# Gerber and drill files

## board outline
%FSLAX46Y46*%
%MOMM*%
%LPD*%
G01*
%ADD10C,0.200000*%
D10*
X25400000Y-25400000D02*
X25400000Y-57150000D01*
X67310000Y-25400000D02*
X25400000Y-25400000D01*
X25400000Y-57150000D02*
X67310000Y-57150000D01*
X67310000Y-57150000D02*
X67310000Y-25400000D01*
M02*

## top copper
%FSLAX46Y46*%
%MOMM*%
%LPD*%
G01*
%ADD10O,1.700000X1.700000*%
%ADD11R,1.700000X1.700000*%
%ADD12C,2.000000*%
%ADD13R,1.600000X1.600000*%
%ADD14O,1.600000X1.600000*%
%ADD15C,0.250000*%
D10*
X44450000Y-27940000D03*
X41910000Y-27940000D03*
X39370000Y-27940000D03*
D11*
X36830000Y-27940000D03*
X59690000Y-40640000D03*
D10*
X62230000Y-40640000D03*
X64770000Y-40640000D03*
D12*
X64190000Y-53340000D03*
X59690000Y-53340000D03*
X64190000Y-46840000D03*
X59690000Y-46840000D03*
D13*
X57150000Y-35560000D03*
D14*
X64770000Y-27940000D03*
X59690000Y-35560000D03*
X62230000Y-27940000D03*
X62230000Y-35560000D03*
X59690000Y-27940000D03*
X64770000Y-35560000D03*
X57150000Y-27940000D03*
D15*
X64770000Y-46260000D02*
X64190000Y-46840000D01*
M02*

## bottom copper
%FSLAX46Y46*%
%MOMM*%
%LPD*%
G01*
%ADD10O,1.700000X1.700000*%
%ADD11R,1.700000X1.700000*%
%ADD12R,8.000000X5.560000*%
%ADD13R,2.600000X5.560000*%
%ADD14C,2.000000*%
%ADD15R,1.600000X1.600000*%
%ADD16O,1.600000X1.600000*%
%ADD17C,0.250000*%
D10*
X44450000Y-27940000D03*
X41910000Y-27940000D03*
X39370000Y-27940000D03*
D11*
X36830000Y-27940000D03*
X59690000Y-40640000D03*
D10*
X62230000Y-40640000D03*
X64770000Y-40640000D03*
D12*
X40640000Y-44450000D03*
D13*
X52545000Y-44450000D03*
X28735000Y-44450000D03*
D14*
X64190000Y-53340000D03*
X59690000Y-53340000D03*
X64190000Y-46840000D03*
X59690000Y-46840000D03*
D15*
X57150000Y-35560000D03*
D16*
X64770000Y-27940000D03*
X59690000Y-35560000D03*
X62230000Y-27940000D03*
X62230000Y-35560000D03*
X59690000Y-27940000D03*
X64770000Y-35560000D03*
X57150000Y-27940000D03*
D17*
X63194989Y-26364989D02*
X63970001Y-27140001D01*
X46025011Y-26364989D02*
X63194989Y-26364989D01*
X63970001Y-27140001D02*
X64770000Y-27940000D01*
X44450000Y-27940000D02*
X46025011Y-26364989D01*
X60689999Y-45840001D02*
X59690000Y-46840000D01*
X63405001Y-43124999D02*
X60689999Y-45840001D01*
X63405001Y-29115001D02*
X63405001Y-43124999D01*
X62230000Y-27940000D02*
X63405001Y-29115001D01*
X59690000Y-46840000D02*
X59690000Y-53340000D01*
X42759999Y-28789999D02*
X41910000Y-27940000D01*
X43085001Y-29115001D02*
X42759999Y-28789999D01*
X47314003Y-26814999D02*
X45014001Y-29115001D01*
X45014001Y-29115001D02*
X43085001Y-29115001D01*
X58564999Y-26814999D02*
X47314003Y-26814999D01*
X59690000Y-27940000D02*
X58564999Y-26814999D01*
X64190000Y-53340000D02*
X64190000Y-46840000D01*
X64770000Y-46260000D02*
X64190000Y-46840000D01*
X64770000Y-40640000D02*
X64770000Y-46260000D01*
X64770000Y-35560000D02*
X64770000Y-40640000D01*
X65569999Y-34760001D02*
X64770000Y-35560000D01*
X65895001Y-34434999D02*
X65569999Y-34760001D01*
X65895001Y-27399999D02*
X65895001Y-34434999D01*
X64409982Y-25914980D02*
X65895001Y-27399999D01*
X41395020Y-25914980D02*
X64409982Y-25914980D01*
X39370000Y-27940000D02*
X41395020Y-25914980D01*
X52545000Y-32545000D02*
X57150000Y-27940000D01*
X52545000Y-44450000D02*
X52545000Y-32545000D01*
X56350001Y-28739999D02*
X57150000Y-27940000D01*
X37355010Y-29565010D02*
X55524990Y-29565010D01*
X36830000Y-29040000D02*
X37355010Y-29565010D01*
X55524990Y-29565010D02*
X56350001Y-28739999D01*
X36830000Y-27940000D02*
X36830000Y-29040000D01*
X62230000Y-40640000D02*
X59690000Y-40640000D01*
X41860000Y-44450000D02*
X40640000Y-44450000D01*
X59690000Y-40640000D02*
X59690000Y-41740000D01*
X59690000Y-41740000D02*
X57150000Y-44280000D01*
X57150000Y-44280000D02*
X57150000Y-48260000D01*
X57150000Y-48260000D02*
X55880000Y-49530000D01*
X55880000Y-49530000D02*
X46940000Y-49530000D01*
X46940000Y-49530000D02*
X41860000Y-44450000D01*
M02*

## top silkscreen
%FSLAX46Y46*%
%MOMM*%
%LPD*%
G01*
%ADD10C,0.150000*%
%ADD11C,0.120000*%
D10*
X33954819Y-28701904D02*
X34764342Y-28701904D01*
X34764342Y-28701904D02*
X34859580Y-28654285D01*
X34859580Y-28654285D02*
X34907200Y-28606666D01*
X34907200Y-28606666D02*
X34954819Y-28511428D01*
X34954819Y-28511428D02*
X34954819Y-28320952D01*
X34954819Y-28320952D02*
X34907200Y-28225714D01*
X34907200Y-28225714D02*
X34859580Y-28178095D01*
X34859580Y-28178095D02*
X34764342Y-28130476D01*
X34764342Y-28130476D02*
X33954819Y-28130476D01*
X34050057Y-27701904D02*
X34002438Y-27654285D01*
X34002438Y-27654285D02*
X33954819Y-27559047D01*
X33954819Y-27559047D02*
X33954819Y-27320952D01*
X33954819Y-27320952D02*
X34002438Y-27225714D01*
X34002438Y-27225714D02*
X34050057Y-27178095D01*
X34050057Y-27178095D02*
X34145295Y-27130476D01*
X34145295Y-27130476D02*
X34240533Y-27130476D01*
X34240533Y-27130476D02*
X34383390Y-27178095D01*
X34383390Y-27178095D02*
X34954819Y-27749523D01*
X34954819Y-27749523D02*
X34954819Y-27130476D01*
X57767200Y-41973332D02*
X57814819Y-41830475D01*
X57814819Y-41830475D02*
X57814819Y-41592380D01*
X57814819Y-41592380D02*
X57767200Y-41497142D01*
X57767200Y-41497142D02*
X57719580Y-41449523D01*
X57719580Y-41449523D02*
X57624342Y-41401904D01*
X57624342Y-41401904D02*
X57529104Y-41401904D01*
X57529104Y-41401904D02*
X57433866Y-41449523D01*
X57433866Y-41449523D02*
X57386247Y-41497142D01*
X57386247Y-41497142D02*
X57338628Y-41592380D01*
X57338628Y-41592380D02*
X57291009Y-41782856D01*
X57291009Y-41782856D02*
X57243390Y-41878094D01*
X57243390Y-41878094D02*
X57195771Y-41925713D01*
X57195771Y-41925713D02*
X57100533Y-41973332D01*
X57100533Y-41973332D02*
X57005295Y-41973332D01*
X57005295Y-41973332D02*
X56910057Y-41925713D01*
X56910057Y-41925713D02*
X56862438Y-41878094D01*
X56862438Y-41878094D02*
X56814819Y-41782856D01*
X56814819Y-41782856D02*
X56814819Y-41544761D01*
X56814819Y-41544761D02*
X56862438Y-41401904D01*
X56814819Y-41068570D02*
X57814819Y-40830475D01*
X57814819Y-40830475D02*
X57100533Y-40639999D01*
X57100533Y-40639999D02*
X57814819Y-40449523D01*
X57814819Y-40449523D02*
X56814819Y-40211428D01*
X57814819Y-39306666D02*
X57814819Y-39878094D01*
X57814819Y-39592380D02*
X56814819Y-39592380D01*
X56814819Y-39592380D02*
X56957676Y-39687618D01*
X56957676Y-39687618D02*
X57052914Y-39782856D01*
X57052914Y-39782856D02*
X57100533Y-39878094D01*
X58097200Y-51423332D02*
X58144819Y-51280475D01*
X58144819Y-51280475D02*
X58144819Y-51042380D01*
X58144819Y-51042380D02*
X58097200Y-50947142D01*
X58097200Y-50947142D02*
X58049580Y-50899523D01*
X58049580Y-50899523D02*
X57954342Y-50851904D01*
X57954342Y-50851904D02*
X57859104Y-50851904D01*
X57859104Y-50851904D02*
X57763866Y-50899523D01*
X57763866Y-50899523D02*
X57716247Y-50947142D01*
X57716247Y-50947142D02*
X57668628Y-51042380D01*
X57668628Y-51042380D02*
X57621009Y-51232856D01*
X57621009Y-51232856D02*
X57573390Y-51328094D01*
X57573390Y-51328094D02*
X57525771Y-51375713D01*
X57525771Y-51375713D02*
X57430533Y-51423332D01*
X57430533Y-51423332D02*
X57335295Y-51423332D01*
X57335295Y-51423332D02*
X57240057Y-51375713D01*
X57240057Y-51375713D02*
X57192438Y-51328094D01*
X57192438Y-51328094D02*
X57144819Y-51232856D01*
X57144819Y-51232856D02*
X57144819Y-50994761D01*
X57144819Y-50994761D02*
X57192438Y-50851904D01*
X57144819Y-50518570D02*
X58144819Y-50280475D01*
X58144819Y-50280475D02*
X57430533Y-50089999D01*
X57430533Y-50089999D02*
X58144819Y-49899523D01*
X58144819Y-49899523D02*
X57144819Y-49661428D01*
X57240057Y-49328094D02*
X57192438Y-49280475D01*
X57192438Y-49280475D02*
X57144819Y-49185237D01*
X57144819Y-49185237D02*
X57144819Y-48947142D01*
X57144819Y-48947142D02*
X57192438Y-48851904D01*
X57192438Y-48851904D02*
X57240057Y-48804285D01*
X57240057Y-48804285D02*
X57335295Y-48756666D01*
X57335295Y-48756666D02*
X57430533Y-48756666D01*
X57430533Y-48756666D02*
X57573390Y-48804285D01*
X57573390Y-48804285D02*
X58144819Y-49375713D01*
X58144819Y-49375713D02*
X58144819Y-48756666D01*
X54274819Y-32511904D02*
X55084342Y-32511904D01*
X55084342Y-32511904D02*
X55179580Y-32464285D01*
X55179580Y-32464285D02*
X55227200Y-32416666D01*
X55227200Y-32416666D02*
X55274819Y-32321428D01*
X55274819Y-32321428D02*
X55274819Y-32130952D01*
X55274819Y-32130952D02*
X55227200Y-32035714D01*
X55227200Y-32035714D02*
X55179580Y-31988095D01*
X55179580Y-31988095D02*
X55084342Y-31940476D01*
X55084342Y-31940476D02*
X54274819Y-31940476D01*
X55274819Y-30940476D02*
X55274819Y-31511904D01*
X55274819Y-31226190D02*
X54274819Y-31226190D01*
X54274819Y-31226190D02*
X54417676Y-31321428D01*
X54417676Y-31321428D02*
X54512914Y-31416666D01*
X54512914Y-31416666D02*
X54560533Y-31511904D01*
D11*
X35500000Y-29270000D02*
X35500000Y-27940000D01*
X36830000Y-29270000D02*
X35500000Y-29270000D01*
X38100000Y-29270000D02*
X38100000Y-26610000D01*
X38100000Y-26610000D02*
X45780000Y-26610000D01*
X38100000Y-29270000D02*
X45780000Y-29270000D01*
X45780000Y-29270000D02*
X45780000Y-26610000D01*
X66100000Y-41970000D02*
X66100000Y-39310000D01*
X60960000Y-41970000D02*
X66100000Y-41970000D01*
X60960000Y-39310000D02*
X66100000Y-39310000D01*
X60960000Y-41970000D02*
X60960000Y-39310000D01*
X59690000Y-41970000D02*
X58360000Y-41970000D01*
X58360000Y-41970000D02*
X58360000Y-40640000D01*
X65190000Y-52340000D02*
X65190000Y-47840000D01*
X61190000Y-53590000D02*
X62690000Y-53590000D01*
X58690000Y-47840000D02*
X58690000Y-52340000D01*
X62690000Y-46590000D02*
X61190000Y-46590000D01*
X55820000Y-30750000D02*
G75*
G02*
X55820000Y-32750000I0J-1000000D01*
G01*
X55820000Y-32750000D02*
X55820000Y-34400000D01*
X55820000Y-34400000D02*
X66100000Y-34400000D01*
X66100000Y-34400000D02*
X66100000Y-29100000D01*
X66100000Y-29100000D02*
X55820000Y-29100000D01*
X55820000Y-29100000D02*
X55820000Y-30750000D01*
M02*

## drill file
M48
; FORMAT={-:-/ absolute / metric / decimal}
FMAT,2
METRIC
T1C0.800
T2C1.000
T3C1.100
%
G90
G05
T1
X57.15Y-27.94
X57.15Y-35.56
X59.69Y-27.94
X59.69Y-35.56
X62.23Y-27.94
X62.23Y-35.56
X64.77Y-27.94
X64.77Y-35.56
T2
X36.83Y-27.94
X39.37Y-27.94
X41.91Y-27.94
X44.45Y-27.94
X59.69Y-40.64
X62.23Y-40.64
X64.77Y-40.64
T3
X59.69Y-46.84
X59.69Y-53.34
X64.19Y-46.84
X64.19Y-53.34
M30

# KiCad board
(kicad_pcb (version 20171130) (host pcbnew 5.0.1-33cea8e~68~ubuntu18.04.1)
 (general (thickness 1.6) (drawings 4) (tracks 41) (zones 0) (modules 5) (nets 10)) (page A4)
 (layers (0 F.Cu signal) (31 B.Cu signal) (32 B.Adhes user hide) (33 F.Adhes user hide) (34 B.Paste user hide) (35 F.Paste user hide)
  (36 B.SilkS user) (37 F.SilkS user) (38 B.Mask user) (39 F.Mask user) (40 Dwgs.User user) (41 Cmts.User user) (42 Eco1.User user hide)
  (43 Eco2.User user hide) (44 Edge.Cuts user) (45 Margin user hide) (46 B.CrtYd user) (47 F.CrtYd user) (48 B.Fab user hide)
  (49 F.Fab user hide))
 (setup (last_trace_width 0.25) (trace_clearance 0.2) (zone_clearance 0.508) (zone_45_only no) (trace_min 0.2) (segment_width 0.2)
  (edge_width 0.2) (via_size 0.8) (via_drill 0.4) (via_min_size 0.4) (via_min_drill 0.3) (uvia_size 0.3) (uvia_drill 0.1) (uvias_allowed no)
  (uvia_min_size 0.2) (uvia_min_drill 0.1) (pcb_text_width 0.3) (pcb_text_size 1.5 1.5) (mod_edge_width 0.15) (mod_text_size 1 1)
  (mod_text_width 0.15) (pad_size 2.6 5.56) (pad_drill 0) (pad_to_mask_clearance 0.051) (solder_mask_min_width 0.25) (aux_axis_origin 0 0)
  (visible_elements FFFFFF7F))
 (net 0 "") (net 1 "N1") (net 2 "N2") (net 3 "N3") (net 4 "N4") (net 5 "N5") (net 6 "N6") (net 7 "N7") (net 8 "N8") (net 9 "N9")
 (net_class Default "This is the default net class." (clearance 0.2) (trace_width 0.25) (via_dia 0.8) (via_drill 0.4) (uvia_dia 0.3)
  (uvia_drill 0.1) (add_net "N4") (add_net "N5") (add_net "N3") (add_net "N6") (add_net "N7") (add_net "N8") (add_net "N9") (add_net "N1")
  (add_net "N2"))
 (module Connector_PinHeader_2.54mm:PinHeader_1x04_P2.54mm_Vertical (layer F.Cu) (at 36.83 27.94 90)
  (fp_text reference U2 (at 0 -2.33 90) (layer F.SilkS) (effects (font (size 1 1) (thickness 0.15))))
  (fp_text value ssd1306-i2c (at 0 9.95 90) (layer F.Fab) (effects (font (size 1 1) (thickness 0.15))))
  (fp_line (start -1.33 -1.33) (end 0 -1.33) (layer F.SilkS) (width 0.12))
  (fp_line (start -1.33 0) (end -1.33 -1.33) (layer F.SilkS) (width 0.12))
  (fp_line (start -1.33 1.27) (end 1.33 1.27) (layer F.SilkS) (width 0.12))
  (fp_line (start 1.33 1.27) (end 1.33 8.95) (layer F.SilkS) (width 0.12))
  (fp_line (start -1.33 1.27) (end -1.33 8.95) (layer F.SilkS) (width 0.12))
  (fp_line (start -1.33 8.95) (end 1.33 8.95) (layer F.SilkS) (width 0.12))
  (pad 4 thru_hole oval (at 0 7.62 90) (size 1.7 1.7) (drill 1) (layers *.Cu *.Mask) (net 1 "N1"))
  (pad 3 thru_hole oval (at 0 5.08 90) (size 1.7 1.7) (drill 1) (layers *.Cu *.Mask) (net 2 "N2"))
  (pad 2 thru_hole oval (at 0 2.54 90) (size 1.7 1.7) (drill 1) (layers *.Cu *.Mask) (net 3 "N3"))
  (pad 1 thru_hole rect (at 0 0 90) (size 1.7 1.7) (drill 1) (layers *.Cu *.Mask) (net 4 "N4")))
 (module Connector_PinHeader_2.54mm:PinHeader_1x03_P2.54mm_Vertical (layer F.Cu) (at 59.69 40.64 90)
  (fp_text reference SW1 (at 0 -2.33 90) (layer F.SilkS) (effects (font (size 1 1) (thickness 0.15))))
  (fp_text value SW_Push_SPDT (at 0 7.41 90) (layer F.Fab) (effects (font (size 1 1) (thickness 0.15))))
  (fp_line (start -1.33 6.41) (end 1.33 6.41) (layer F.SilkS) (width 0.12))
  (fp_line (start -1.33 1.27) (end -1.33 6.41) (layer F.SilkS) (width 0.12))
  (fp_line (start 1.33 1.27) (end 1.33 6.41) (layer F.SilkS) (width 0.12))
  (fp_line (start -1.33 1.27) (end 1.33 1.27) (layer F.SilkS) (width 0.12))
  (fp_line (start -1.33 0) (end -1.33 -1.33) (layer F.SilkS) (width 0.12))
  (fp_line (start -1.33 -1.33) (end 0 -1.33) (layer F.SilkS) (width 0.12))
  (pad 1 thru_hole rect (at 0 0 90) (size 1.7 1.7) (drill 1) (layers *.Cu *.Mask) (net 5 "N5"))
  (pad 2 thru_hole oval (at 0 2.54 90) (size 1.7 1.7) (drill 1) (layers *.Cu *.Mask) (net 5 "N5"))
  (pad 3 thru_hole oval (at 0 5.08 90) (size 1.7 1.7) (drill 1) (layers *.Cu *.Mask) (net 3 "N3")))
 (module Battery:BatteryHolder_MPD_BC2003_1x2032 (layer B.Cu) (at 40.64 44.45)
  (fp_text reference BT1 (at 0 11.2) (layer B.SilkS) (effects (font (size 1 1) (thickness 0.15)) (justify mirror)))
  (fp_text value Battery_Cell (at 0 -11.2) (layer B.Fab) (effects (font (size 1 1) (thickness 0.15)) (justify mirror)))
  (pad 2 smd rect (at 0 0) (size 8 5.56) (layers B.Cu B.Paste B.Mask) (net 5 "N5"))
  (pad 1 smd rect (at 11.905 0) (size 2.6 5.56) (layers B.Cu B.Paste B.Mask) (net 4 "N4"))
  (pad 1 smd rect (at -11.905 0) (size 2.6 5.56) (layers B.Cu B.Paste B.Mask) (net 4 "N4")))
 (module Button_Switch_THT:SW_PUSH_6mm (layer F.Cu) (at 59.69 53.34 90)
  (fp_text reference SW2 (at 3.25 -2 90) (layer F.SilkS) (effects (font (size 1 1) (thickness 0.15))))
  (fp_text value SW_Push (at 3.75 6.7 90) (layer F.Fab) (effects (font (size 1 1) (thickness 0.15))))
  (fp_line (start 1 5.5) (end 5.5 5.5) (layer F.SilkS) (width 0.12))
  (fp_line (start -0.25 1.5) (end -0.25 3) (layer F.SilkS) (width 0.12))
  (fp_line (start 5.5 -1) (end 1 -1) (layer F.SilkS) (width 0.12))
  (fp_line (start 6.75 3) (end 6.75 1.5) (layer F.SilkS) (width 0.12))
  (pad 2 thru_hole circle (at 0 4.5 180) (size 2 2) (drill 1.1) (layers *.Cu *.Mask) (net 3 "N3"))
  (pad 1 thru_hole circle (at 0 0 180) (size 2 2) (drill 1.1) (layers *.Cu *.Mask) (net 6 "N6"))
  (pad 2 thru_hole circle (at 6.5 4.5 180) (size 2 2) (drill 1.1) (layers *.Cu *.Mask) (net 3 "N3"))
  (pad 1 thru_hole circle (at 6.5 0 180) (size 2 2) (drill 1.1) (layers *.Cu *.Mask) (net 6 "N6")))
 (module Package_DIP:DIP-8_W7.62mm (layer F.Cu) (at 57.15 35.56 90)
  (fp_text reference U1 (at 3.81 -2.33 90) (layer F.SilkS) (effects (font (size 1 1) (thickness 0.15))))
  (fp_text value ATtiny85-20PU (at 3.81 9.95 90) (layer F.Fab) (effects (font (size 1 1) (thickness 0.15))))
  (fp_arc (start 3.81 -1.33) (end 2.81 -1.33) (angle -180) (layer F.SilkS) (width 0.12))
  (fp_line (start 2.81 -1.33) (end 1.16 -1.33) (layer F.SilkS) (width 0.12))
  (fp_line (start 1.16 -1.33) (end 1.16 8.95) (layer F.SilkS) (width 0.12))
  (fp_line (start 1.16 8.95) (end 6.46 8.95) (layer F.SilkS) (width 0.12))
  (fp_line (start 6.46 8.95) (end 6.46 -1.33) (layer F.SilkS) (width 0.12))
  (fp_line (start 6.46 -1.33) (end 4.81 -1.33) (layer F.SilkS) (width 0.12))
  (pad 1 thru_hole rect (at 0 0 90) (size 1.6 1.6) (drill 0.8) (layers *.Cu *.Mask) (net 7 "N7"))
  (pad 5 thru_hole oval (at 7.62 7.62 90) (size 1.6 1.6) (drill 0.8) (layers *.Cu *.Mask) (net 1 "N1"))
  (pad 2 thru_hole oval (at 0 2.54 90) (size 1.6 1.6) (drill 0.8) (layers *.Cu *.Mask) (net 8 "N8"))
  (pad 6 thru_hole oval (at 7.62 5.08 90) (size 1.6 1.6) (drill 0.8) (layers *.Cu *.Mask) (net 6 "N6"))
  (pad 3 thru_hole oval (at 0 5.08 90) (size 1.6 1.6) (drill 0.8) (layers *.Cu *.Mask) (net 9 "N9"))
  (pad 7 thru_hole oval (at 7.62 2.54 90) (size 1.6 1.6) (drill 0.8) (layers *.Cu *.Mask) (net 2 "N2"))
  (pad 4 thru_hole oval (at 0 7.62 90) (size 1.6 1.6) (drill 0.8) (layers *.Cu *.Mask) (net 3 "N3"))
  (pad 8 thru_hole oval (at 7.62 0 90) (size 1.6 1.6) (drill 0.8) (layers *.Cu *.Mask) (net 4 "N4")))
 (gr_line (start 25.4 25.4) (end 25.4 57.15) (layer Edge.Cuts) (width 0.2))
 (gr_line (start 67.31 25.4) (end 25.4 25.4) (layer Edge.Cuts) (width 0.2))
 (gr_line (start 25.4 57.15) (end 67.31 57.15) (layer Edge.Cuts) (width 0.2))
 (gr_line (start 67.31 57.15) (end 67.31 25.4) (layer Edge.Cuts) (width 0.2))
 (segment (start 63.194989 26.364989) (end 63.970001 27.140001) (width 0.25) (layer B.Cu) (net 1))
 (segment (start 46.025011 26.364989) (end 63.194989 26.364989) (width 0.25) (layer B.Cu) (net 1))
 (segment (start 63.970001 27.140001) (end 64.77 27.94) (width 0.25) (layer B.Cu) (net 1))
 (segment (start 44.45 27.94) (end 46.025011 26.364989) (width 0.25) (layer B.Cu) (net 1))
 (segment (start 60.689999 45.840001) (end 59.69 46.84) (width 0.25) (layer B.Cu) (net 6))
 (segment (start 63.405001 43.124999) (end 60.689999 45.840001) (width 0.25) (layer B.Cu) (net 6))
 (segment (start 63.405001 29.115001) (end 63.405001 43.124999) (width 0.25) (layer B.Cu) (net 6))
 (segment (start 62.23 27.94) (end 63.405001 29.115001) (width 0.25) (layer B.Cu) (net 6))
 (segment (start 59.69 46.84) (end 59.69 53.34) (width 0.25) (layer B.Cu) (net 6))
 (segment (start 42.759999 28.789999) (end 41.91 27.94) (width 0.25) (layer B.Cu) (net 2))
 (segment (start 43.085001 29.115001) (end 42.759999 28.789999) (width 0.25) (layer B.Cu) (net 2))
 (segment (start 47.314003 26.814999) (end 45.014001 29.115001) (width 0.25) (layer B.Cu) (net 2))
 (segment (start 45.014001 29.115001) (end 43.085001 29.115001) (width 0.25) (layer B.Cu) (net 2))
 (segment (start 58.564999 26.814999) (end 47.314003 26.814999) (width 0.25) (layer B.Cu) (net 2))
 (segment (start 59.69 27.94) (end 58.564999 26.814999) (width 0.25) (layer B.Cu) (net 2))
 (segment (start 64.77 46.26) (end 64.19 46.84) (width 0.25) (layer F.Cu) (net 3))
 (segment (start 64.19 53.34) (end 64.19 46.84) (width 0.25) (layer B.Cu) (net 3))
 (segment (start 64.77 46.26) (end 64.19 46.84) (width 0.25) (layer B.Cu) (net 3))
 (segment (start 64.77 40.64) (end 64.77 46.26) (width 0.25) (layer B.Cu) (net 3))
 (segment (start 64.77 35.56) (end 64.77 40.64) (width 0.25) (layer B.Cu) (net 3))
 (segment (start 65.569999 34.760001) (end 64.77 35.56) (width 0.25) (layer B.Cu) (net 3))
 (segment (start 65.895001 34.434999) (end 65.569999 34.760001) (width 0.25) (layer B.Cu) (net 3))
 (segment (start 65.895001 27.399999) (end 65.895001 34.434999) (width 0.25) (layer B.Cu) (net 3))
 (segment (start 64.409982 25.91498) (end 65.895001 27.399999) (width 0.25) (layer B.Cu) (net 3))
 (segment (start 41.39502 25.91498) (end 64.409982 25.91498) (width 0.25) (layer B.Cu) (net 3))
 (segment (start 39.37 27.94) (end 41.39502 25.91498) (width 0.25) (layer B.Cu) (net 3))
 (segment (start 52.545 32.545) (end 57.15 27.94) (width 0.25) (layer B.Cu) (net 4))
 (segment (start 52.545 44.45) (end 52.545 32.545) (width 0.25) (layer B.Cu) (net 4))
 (segment (start 56.350001 28.739999) (end 57.15 27.94) (width 0.25) (layer B.Cu) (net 4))
 (segment (start 37.35501 29.56501) (end 55.52499 29.56501) (width 0.25) (layer B.Cu) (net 4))
 (segment (start 36.83 29.04) (end 37.35501 29.56501) (width 0.25) (layer B.Cu) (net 4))
 (segment (start 55.52499 29.56501) (end 56.350001 28.739999) (width 0.25) (layer B.Cu) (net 4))
 (segment (start 36.83 27.94) (end 36.83 29.04) (width 0.25) (layer B.Cu) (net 4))
 (segment (start 62.23 40.64) (end 59.69 40.64) (width 0.25) (layer B.Cu) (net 5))
 (segment (start 41.86 44.45) (end 40.64 44.45) (width 0.25) (layer B.Cu) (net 5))
 (segment (start 59.69 40.64) (end 59.69 41.74) (width 0.25) (layer B.Cu) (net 5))
 (segment (start 59.69 41.74) (end 57.15 44.28) (width 0.25) (layer B.Cu) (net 5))
 (segment (start 57.15 44.28) (end 57.15 48.26) (width 0.25) (layer B.Cu) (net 5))
 (segment (start 57.15 48.26) (end 55.88 49.53) (width 0.25) (layer B.Cu) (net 5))
 (segment (start 55.88 49.53) (end 46.94 49.53) (width 0.25) (layer B.Cu) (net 5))
 (segment (start 46.94 49.53) (end 41.86 44.45) (width 0.25) (layer B.Cu) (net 5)))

